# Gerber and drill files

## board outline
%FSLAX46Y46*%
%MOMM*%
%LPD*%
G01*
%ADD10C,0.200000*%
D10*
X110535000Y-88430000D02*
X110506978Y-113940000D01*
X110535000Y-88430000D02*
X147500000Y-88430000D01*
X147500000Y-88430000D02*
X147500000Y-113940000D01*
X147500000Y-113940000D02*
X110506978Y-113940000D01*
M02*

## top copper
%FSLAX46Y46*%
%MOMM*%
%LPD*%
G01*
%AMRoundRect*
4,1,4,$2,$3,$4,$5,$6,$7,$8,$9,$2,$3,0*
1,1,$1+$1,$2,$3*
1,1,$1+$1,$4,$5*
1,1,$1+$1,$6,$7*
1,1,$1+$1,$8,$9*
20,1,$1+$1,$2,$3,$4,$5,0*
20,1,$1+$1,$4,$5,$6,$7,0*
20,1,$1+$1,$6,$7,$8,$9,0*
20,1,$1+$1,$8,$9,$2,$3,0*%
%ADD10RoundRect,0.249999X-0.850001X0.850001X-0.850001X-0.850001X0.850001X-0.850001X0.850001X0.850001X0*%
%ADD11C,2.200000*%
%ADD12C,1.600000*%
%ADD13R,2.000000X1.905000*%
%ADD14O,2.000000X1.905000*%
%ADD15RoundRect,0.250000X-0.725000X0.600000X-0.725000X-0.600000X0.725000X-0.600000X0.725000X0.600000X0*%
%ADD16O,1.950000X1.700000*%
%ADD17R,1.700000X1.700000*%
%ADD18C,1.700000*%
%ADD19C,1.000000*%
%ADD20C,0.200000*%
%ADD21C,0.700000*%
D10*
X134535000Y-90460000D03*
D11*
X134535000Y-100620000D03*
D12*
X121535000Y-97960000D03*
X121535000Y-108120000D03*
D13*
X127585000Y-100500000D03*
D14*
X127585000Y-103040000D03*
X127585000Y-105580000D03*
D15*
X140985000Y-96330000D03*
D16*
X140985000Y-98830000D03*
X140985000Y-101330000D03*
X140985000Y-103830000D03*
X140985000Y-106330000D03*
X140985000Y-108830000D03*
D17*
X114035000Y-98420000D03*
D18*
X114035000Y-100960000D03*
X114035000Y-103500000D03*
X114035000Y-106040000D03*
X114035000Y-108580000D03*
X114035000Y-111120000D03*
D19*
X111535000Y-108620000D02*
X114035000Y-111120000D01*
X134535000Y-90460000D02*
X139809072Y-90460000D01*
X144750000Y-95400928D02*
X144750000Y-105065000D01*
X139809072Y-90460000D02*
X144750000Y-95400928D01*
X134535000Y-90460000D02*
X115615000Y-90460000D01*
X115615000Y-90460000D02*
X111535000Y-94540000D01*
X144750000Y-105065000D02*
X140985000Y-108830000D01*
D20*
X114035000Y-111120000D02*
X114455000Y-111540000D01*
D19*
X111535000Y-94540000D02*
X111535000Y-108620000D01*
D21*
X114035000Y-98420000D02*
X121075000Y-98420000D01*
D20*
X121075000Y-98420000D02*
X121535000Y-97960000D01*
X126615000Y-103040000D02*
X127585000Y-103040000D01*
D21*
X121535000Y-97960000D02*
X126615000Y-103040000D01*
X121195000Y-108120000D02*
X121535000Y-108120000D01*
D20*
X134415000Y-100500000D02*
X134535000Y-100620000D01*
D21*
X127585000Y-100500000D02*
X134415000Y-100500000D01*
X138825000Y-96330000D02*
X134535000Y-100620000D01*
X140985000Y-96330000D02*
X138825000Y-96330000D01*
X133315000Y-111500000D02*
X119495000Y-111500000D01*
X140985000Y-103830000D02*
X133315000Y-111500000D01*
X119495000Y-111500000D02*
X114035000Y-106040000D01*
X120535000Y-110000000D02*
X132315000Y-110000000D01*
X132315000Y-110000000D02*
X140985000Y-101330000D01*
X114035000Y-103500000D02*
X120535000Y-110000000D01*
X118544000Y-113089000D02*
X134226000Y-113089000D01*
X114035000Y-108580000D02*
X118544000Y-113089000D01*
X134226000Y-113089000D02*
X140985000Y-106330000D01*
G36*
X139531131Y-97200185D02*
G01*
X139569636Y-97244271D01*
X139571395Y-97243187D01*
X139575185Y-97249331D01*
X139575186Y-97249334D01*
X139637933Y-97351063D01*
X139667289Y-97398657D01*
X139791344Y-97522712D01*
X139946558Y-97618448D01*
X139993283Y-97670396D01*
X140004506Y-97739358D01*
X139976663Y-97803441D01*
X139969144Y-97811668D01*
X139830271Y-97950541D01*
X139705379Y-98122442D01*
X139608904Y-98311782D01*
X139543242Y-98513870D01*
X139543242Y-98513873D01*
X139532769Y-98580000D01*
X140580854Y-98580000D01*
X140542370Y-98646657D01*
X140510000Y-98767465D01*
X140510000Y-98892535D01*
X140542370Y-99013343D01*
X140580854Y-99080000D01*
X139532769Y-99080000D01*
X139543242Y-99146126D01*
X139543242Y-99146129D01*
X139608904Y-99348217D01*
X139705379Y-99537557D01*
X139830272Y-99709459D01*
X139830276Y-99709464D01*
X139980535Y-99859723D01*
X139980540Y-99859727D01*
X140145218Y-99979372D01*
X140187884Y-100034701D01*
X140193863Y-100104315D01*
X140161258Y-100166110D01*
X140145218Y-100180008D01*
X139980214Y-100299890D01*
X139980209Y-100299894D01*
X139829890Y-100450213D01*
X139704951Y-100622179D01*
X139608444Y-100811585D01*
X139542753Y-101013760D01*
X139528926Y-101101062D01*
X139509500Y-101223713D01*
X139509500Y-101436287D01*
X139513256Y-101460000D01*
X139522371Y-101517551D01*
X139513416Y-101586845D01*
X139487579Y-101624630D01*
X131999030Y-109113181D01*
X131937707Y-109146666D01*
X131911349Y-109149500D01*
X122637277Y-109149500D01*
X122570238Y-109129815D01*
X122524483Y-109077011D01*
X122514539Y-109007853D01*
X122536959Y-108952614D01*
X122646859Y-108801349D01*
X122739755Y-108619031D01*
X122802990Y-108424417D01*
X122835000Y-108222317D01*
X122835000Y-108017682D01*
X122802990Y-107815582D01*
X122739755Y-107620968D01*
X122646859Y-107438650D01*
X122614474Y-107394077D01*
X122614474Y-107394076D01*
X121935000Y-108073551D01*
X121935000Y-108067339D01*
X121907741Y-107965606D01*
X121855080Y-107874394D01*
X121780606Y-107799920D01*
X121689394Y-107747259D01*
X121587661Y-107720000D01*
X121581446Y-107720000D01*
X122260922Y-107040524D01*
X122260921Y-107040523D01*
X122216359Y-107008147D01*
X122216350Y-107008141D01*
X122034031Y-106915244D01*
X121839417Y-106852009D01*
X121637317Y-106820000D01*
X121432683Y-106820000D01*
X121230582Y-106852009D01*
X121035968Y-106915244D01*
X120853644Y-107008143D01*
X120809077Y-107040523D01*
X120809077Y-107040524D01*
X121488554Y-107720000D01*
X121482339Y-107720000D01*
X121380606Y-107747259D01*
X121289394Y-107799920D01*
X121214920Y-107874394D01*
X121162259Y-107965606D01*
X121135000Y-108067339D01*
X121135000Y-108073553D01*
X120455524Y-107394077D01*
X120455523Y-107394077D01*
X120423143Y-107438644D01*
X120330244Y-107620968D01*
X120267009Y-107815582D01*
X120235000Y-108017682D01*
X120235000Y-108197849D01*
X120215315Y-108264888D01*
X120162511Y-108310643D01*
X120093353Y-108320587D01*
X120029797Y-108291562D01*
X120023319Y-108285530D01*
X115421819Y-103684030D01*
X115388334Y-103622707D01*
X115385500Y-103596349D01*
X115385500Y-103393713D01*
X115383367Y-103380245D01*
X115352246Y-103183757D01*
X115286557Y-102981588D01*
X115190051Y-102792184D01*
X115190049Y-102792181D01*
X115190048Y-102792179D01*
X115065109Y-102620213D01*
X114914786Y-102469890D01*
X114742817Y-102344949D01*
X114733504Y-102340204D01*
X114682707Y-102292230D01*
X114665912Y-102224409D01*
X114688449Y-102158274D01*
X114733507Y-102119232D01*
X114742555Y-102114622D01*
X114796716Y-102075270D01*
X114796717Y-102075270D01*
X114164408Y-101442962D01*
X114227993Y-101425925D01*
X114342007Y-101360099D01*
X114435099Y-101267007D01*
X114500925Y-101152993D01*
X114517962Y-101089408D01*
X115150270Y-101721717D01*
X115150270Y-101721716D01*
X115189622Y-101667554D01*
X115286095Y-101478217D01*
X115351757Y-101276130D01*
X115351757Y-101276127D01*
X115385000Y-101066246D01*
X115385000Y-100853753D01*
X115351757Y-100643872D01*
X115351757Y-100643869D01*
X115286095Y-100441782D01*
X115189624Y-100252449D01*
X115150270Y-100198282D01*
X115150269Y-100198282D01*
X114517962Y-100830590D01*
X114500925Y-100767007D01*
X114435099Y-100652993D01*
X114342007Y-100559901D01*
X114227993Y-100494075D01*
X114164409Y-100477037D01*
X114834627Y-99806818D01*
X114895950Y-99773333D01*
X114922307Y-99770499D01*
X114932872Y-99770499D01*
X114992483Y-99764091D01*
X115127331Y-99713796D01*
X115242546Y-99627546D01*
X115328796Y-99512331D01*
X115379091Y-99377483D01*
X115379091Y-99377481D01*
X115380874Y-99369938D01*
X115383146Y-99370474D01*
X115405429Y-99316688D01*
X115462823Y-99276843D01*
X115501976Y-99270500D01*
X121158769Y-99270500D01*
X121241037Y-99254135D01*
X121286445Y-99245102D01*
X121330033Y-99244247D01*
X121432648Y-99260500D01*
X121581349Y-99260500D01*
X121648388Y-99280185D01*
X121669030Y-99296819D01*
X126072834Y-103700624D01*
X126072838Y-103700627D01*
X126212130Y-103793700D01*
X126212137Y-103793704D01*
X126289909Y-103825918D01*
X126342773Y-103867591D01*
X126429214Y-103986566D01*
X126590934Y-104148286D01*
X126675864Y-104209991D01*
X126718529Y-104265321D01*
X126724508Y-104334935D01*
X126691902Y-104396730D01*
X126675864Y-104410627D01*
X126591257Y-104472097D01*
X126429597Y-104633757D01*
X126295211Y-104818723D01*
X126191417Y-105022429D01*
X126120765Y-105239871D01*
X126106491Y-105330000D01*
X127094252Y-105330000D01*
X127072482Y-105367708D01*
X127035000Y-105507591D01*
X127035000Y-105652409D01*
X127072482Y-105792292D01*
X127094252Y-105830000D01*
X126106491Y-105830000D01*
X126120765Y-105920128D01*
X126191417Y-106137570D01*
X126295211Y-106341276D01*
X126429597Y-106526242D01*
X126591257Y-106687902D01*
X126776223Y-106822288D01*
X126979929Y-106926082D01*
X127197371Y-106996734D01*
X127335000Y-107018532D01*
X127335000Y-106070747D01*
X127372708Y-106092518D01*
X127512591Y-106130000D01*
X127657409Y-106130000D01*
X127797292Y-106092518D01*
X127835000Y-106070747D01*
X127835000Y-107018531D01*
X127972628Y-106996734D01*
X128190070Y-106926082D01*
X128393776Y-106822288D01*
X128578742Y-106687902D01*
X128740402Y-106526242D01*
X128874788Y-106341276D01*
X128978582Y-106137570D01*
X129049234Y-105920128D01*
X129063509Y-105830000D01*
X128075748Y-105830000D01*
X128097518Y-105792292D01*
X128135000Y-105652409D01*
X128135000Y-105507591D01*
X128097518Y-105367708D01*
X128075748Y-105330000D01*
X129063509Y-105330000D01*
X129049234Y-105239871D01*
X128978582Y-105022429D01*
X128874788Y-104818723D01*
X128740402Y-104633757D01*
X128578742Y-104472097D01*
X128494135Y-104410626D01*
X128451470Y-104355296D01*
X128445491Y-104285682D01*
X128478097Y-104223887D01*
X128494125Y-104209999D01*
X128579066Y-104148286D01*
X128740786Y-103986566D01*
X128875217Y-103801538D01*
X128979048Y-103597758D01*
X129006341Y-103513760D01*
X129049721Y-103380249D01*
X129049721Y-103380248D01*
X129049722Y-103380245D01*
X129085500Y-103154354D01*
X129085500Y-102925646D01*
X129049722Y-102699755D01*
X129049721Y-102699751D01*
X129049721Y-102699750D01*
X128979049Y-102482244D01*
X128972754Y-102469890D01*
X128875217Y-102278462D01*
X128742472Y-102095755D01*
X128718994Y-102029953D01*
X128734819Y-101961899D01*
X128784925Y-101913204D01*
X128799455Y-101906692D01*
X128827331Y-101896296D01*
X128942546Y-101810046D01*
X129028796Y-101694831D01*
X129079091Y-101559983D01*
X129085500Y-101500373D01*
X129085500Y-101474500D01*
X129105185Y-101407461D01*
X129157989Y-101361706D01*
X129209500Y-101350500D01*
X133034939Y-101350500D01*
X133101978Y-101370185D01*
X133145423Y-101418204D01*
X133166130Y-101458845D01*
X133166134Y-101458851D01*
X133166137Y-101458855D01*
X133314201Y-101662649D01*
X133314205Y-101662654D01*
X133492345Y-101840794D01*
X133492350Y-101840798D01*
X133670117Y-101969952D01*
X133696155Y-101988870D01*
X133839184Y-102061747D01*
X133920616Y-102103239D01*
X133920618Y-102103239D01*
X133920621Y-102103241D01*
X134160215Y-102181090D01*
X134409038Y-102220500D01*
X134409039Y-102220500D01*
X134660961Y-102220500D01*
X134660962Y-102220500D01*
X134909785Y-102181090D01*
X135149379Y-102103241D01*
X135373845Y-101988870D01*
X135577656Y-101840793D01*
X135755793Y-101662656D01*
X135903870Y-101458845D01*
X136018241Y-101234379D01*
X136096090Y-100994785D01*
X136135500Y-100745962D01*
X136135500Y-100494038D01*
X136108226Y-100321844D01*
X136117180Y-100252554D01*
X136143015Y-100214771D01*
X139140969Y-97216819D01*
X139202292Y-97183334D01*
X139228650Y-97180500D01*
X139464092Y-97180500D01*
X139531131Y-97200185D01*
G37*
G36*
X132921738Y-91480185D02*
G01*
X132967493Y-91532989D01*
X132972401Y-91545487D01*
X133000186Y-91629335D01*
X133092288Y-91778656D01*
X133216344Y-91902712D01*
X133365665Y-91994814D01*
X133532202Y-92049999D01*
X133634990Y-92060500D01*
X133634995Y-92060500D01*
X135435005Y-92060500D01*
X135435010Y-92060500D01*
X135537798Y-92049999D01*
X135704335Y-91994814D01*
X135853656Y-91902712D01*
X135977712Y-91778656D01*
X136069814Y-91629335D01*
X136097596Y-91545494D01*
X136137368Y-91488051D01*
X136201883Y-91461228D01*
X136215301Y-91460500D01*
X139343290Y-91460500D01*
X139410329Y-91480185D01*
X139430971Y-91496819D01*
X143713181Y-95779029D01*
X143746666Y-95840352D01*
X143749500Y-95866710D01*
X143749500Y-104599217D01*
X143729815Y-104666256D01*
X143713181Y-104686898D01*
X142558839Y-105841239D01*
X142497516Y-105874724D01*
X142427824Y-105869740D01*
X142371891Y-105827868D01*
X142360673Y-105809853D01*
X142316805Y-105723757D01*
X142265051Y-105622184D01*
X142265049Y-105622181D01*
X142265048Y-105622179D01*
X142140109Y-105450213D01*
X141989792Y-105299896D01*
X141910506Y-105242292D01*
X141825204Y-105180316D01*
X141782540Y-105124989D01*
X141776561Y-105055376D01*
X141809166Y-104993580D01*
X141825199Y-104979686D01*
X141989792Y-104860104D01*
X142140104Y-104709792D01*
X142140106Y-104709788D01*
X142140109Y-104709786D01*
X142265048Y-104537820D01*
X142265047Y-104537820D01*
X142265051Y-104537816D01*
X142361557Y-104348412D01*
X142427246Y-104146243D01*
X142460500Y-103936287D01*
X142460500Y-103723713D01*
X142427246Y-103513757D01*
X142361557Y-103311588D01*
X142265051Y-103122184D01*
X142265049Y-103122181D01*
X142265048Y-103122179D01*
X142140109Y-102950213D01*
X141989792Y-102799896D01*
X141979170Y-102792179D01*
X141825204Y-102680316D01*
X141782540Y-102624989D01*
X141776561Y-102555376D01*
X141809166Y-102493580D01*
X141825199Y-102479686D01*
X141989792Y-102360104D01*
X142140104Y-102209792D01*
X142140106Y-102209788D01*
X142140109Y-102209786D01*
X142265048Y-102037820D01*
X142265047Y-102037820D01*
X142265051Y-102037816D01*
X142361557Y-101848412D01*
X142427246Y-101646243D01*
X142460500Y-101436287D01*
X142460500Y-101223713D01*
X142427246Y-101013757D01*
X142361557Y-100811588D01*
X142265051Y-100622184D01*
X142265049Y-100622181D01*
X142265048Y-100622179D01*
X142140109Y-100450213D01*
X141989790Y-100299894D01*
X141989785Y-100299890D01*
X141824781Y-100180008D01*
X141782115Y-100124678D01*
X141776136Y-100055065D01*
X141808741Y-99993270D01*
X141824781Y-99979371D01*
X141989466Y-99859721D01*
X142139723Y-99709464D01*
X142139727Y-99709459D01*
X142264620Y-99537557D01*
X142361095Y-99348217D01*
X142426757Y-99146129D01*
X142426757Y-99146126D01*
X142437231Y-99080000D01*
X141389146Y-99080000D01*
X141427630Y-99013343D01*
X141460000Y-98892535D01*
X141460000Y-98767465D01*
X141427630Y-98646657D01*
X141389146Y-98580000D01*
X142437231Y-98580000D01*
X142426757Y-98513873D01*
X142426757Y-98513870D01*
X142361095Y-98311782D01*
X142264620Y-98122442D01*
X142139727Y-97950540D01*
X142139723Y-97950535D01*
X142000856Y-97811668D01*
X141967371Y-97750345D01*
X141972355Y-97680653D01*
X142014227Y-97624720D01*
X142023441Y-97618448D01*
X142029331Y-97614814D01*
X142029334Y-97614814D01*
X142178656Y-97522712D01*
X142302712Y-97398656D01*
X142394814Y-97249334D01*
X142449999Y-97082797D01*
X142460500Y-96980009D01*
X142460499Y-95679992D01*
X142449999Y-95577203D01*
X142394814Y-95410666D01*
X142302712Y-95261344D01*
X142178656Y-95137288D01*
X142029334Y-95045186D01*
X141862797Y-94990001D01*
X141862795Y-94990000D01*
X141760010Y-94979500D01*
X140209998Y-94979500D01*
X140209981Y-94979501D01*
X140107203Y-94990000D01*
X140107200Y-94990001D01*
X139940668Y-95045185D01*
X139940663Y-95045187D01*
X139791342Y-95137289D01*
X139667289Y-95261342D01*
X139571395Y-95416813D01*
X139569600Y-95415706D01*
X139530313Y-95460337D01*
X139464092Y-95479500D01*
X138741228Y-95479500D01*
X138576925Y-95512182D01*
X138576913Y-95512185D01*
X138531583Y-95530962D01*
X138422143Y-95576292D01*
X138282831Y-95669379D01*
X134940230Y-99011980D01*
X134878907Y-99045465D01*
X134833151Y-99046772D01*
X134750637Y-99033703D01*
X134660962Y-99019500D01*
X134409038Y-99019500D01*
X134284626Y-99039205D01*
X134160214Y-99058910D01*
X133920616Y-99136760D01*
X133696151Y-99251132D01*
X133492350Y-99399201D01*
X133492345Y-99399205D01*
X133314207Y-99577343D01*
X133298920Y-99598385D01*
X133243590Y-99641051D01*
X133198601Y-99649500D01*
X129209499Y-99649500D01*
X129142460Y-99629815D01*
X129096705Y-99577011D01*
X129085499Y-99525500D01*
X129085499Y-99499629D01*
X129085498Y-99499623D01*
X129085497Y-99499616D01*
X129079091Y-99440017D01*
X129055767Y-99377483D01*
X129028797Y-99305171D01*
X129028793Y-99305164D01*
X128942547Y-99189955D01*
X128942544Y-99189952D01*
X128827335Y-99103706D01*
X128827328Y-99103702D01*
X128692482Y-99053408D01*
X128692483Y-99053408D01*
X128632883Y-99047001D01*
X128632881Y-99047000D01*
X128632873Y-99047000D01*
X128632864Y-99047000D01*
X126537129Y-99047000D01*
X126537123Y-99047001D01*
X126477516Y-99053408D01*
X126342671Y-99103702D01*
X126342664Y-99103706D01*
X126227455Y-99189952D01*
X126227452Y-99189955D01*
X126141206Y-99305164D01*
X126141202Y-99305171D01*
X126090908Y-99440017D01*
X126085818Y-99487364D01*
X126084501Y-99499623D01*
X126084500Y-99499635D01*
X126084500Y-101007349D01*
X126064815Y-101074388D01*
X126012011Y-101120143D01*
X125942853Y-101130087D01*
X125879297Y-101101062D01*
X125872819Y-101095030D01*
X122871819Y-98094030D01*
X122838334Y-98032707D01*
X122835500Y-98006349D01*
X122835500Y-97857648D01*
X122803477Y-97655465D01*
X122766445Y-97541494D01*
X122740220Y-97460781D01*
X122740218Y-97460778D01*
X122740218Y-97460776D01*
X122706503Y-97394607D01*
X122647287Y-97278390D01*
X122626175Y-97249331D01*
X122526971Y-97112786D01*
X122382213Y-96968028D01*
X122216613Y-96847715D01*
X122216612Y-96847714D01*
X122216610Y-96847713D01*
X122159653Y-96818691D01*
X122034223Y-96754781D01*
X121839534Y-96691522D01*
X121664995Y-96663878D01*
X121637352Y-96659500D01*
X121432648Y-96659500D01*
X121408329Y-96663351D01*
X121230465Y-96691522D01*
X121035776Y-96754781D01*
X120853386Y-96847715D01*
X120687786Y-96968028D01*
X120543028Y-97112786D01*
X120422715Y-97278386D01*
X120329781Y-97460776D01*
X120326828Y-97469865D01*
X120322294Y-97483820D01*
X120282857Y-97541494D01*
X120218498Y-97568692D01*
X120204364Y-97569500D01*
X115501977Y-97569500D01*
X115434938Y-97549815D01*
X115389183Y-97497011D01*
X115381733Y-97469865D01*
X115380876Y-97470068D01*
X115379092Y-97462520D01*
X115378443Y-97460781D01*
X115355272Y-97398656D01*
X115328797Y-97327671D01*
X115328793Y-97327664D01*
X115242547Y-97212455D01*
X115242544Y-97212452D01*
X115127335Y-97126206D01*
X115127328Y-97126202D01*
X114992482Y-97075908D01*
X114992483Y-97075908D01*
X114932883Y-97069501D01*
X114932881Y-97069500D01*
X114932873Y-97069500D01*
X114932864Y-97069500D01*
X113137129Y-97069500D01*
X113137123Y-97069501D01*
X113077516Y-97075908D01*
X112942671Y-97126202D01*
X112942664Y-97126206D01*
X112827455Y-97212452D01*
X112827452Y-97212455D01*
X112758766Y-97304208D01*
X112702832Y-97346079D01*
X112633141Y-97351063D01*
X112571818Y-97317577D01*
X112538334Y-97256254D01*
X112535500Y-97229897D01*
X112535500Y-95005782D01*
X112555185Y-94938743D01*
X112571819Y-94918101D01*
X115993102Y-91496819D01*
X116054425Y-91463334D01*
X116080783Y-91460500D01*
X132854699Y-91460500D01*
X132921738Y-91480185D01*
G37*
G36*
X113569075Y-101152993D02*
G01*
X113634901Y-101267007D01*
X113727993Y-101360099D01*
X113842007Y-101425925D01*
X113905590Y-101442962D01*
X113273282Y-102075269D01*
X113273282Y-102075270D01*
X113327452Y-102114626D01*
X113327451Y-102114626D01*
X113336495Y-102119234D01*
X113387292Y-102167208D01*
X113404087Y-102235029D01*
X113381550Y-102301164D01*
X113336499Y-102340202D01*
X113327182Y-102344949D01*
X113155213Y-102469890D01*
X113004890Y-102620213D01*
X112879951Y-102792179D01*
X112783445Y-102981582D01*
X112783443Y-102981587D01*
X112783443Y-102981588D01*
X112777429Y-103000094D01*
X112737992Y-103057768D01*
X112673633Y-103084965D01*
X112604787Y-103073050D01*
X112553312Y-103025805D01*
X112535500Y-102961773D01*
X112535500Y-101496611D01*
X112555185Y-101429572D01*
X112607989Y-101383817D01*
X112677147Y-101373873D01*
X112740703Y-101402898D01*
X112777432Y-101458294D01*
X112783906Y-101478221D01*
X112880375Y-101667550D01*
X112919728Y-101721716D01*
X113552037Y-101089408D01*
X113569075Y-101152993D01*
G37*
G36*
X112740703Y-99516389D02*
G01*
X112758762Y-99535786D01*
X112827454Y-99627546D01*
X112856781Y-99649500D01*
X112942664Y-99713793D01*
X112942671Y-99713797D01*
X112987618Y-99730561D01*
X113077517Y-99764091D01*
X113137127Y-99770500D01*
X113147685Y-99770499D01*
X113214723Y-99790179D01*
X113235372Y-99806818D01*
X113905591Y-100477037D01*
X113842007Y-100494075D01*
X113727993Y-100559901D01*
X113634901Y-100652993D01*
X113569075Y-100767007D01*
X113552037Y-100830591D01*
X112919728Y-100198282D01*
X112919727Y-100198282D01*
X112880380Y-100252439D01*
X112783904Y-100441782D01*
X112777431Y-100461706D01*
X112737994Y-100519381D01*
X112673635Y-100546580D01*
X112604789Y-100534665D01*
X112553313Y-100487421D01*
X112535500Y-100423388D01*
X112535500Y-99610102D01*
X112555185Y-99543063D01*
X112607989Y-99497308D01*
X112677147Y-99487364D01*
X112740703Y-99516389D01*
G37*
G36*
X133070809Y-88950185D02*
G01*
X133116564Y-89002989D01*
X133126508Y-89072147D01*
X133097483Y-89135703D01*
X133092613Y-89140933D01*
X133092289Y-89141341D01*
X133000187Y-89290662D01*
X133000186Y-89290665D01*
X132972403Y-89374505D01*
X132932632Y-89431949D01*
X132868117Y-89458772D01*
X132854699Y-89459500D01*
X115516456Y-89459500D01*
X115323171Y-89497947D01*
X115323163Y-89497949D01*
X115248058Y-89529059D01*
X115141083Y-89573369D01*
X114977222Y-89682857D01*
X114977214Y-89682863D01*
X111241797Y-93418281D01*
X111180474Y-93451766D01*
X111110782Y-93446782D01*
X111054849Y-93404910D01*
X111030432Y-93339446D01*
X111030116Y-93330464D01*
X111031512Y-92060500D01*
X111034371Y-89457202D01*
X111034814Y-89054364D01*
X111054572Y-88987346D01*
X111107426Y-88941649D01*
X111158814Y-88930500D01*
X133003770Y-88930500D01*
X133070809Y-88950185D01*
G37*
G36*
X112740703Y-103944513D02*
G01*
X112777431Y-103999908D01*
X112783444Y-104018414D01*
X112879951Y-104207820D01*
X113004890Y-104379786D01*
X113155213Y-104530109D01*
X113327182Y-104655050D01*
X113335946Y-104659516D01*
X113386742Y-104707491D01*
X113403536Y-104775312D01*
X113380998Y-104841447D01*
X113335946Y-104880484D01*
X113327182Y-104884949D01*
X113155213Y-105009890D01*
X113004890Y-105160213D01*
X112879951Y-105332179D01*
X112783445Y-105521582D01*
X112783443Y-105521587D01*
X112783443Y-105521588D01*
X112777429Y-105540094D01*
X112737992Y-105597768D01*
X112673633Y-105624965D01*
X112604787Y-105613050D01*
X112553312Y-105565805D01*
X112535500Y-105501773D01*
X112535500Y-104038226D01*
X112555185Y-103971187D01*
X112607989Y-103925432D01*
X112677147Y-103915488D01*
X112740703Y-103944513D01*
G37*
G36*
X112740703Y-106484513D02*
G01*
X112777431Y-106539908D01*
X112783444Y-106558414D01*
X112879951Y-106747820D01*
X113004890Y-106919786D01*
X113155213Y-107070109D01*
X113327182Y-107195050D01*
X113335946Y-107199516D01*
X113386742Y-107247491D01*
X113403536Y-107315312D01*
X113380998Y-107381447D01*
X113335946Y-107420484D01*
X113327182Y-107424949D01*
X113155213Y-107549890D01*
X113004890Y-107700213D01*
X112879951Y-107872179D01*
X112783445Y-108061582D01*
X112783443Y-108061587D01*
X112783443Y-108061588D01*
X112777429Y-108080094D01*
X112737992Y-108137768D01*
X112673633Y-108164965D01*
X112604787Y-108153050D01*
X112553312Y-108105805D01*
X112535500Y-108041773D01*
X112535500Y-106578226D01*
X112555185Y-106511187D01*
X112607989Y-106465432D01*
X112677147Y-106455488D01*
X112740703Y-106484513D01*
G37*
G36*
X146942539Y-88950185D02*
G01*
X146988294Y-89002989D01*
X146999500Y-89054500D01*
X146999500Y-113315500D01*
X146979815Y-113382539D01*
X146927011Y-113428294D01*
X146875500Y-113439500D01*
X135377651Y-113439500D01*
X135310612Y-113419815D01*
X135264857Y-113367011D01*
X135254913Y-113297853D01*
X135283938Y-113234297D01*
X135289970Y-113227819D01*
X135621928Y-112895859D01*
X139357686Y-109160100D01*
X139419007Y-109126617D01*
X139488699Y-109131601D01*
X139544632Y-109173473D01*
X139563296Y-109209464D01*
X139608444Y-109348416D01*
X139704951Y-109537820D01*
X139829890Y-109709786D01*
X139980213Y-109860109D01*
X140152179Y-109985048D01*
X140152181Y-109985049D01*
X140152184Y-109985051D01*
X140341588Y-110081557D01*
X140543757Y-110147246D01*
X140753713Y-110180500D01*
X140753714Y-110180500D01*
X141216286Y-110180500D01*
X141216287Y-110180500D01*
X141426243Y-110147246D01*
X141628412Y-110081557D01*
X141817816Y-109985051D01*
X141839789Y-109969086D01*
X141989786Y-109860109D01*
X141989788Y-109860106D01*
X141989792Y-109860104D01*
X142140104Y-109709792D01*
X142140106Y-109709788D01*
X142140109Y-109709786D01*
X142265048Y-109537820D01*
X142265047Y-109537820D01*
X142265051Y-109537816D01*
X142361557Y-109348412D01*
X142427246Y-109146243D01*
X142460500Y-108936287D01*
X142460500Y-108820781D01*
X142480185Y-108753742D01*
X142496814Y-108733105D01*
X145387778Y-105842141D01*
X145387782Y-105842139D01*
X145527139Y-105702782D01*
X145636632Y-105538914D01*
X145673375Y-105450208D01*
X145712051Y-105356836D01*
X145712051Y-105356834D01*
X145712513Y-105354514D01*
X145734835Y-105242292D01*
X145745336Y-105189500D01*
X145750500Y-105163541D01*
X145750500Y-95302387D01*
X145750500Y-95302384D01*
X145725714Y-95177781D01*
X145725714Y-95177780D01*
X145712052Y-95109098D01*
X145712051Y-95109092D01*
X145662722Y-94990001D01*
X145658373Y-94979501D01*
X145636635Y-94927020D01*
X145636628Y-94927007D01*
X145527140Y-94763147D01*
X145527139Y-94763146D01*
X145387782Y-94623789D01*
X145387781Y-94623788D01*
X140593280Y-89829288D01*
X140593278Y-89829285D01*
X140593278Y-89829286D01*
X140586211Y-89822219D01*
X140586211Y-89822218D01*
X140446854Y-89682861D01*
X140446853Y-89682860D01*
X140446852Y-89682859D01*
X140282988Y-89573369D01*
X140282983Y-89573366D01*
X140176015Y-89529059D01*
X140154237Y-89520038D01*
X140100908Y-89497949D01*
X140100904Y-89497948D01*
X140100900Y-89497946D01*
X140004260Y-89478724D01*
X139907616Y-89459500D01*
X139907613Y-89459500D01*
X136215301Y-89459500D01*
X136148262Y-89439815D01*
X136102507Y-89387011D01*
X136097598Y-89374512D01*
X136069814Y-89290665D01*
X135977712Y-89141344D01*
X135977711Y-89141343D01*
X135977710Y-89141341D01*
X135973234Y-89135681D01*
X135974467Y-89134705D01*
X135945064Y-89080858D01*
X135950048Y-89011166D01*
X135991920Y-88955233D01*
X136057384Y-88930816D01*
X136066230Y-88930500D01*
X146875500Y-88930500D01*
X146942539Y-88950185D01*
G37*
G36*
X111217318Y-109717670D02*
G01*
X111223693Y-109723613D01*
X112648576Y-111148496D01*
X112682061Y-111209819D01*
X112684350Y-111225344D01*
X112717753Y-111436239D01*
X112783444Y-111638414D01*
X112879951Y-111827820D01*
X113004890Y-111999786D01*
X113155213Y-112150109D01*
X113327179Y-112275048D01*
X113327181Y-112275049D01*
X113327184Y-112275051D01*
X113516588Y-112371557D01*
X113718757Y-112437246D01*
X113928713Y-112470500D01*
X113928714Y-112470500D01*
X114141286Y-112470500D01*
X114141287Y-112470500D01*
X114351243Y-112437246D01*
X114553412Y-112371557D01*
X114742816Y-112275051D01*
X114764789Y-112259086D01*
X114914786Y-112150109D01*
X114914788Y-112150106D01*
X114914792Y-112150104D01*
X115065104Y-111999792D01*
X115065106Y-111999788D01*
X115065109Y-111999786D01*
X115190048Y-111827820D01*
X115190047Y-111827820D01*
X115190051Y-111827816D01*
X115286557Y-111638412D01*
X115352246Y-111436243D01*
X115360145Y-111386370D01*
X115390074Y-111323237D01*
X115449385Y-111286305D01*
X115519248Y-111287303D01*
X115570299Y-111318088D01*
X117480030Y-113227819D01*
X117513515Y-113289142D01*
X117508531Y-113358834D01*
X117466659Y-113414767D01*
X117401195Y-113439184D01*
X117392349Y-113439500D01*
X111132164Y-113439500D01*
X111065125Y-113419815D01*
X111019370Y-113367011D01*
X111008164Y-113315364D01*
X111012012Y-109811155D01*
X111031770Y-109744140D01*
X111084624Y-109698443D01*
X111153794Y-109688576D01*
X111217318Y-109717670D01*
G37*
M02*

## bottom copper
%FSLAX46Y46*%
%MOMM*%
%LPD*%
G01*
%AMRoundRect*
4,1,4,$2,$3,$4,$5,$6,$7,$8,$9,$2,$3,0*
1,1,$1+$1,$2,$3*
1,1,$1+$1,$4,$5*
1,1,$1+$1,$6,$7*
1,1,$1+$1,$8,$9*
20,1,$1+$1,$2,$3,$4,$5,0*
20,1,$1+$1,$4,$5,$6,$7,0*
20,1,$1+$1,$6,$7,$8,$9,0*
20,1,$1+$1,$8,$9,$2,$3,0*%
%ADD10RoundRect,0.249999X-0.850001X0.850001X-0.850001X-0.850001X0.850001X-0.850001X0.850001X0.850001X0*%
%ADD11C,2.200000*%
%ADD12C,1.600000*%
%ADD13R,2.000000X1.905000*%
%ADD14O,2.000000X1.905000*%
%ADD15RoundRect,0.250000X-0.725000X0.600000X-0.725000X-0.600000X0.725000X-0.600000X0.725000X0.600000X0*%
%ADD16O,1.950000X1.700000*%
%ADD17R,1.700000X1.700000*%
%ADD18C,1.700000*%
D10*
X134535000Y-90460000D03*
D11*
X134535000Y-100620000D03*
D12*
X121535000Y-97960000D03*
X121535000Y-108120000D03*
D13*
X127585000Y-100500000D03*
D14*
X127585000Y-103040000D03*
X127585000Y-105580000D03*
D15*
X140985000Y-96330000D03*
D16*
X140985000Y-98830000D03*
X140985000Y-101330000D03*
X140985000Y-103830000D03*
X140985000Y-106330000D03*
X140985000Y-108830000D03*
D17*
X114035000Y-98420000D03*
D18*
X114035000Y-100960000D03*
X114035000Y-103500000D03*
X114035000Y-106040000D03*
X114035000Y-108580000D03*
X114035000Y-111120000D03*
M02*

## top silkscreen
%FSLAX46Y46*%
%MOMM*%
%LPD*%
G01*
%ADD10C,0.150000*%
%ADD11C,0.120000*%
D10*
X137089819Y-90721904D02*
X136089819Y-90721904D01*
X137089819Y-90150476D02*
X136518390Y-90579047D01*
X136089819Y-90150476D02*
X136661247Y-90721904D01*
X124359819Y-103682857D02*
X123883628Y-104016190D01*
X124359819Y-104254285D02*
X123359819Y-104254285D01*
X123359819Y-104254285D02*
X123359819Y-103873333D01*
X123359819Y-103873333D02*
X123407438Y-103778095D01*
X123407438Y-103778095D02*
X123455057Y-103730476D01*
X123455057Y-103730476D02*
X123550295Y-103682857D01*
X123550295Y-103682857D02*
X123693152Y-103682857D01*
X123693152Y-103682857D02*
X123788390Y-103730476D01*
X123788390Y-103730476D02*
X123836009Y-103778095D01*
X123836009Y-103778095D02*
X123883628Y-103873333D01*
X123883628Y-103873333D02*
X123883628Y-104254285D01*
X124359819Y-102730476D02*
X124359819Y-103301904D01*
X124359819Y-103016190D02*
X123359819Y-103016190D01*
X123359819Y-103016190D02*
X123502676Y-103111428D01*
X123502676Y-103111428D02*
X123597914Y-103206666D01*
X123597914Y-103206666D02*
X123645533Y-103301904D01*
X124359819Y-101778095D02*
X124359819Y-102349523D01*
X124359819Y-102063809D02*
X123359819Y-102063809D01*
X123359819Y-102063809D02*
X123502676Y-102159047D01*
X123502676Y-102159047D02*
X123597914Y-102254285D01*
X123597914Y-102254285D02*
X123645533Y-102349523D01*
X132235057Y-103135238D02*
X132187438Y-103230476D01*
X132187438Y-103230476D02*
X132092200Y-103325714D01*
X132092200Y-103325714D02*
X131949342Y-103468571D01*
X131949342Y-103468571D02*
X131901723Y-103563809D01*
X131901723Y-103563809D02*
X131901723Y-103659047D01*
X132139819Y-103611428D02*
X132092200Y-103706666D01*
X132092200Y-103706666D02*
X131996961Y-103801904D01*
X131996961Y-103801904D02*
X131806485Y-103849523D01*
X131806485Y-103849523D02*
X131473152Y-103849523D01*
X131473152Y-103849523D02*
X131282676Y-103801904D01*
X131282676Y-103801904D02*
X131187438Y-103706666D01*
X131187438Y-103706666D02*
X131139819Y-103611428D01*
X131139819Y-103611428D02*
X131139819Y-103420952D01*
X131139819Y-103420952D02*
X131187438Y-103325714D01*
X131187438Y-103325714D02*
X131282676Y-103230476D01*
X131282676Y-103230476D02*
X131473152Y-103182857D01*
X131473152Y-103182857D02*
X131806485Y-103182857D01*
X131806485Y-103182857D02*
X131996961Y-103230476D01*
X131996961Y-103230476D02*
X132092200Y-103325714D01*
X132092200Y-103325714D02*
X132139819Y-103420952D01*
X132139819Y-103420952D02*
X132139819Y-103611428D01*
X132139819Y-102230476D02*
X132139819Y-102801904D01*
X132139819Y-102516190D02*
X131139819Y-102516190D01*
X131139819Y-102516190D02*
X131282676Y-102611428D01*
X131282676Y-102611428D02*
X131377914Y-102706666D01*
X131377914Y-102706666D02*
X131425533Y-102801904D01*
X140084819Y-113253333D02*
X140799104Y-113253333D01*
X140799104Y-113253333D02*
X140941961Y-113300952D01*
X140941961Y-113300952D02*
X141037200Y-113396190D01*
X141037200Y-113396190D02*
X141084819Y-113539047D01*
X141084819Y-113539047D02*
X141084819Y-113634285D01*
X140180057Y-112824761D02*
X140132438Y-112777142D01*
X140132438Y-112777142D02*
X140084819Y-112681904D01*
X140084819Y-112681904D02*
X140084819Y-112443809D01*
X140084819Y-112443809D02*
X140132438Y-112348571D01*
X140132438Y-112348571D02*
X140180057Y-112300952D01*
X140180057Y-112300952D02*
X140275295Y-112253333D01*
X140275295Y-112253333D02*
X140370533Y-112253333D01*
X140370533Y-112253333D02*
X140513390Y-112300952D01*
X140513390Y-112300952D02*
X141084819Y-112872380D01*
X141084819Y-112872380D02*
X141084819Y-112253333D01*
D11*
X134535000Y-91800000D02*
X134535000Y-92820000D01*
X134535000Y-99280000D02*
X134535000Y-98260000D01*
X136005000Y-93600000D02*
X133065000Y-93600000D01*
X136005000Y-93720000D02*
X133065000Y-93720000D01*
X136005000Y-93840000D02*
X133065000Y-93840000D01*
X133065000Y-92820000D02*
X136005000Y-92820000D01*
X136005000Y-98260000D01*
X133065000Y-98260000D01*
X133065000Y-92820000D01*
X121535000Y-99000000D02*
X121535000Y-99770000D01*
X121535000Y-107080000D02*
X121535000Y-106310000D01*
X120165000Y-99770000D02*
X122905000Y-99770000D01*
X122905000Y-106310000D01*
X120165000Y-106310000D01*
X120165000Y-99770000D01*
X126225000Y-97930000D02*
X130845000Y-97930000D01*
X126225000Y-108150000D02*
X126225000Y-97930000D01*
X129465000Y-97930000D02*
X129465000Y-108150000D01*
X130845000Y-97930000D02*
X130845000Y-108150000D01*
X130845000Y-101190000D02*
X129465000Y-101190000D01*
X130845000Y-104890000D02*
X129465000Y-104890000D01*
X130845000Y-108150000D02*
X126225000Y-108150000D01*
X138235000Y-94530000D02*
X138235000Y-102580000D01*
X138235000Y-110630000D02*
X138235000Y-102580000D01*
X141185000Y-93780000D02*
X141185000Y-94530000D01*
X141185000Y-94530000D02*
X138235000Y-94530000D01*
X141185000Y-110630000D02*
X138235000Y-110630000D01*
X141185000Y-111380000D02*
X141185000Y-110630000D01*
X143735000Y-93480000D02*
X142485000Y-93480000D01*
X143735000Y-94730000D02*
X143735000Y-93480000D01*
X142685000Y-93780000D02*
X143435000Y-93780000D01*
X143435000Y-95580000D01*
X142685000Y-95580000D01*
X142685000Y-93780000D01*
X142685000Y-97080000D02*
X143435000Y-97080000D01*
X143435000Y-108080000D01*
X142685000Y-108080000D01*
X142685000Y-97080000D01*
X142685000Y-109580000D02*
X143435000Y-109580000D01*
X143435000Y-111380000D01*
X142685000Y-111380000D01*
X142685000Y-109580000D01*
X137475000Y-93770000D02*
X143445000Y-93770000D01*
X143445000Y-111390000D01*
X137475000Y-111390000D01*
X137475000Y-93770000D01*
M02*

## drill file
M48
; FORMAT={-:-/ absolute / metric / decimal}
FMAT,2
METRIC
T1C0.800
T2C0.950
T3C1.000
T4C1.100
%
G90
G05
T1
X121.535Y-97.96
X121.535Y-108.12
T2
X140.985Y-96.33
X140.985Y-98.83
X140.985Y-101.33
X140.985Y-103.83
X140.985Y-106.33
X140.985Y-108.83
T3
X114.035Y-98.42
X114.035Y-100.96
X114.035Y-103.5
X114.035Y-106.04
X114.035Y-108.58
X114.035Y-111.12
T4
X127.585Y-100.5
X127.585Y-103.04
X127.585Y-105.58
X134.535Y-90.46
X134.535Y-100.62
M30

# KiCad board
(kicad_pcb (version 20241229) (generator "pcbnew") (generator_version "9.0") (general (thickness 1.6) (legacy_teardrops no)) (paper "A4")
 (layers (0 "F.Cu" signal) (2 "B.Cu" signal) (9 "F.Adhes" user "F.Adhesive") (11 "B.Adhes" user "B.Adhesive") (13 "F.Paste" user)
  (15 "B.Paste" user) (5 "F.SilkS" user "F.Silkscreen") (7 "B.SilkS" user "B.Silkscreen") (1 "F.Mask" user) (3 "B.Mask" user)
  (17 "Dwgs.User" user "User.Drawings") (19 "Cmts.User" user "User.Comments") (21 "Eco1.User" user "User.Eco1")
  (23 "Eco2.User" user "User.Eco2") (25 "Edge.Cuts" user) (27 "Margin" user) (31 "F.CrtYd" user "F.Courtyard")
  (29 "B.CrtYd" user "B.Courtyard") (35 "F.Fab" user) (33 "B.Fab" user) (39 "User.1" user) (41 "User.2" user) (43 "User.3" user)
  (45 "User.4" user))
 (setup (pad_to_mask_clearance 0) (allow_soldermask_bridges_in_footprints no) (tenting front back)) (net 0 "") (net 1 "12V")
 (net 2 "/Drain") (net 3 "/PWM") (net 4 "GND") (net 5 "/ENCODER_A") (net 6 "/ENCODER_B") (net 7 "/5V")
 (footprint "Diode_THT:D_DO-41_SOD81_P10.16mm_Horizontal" (layer "F.Cu") (at 134.535 90.46 -90)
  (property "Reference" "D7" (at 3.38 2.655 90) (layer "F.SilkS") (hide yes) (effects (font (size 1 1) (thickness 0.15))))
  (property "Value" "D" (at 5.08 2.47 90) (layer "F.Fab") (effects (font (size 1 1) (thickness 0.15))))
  (fp_line (start 1.34 0) (end 2.36 0) (stroke (width 0.12) (type solid)) (layer "F.SilkS"))
  (fp_line (start 8.82 0) (end 7.8 0) (stroke (width 0.12) (type solid)) (layer "F.SilkS"))
  (fp_line (start 3.14 -1.47) (end 3.14 1.47) (stroke (width 0.12) (type solid)) (layer "F.SilkS"))
  (fp_line (start 3.26 -1.47) (end 3.26 1.47) (stroke (width 0.12) (type solid)) (layer "F.SilkS"))
  (fp_line (start 3.38 -1.47) (end 3.38 1.47) (stroke (width 0.12) (type solid)) (layer "F.SilkS"))
  (fp_rect (start 2.36 -1.47) (end 7.8 1.47) (stroke (width 0.12) (type solid)) (fill no) (layer "F.SilkS"))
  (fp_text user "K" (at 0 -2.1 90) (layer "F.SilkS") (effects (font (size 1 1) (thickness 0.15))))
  (pad "1" thru_hole roundrect (at 0 0 270) (size 2.2 2.2) (drill 1.1) (layers "*.Cu" "*.Mask") (remove_unused_layers no)
   (roundrect_rratio 0.113636) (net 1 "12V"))
  (pad "2" thru_hole circle (at 10.16 0 270) (size 2.2 2.2) (drill 1.1) (layers "*.Cu" "*.Mask") (remove_unused_layers no) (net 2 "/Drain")))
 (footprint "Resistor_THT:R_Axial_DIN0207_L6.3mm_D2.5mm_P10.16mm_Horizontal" (layer "F.Cu") (at 121.535 97.96 -90)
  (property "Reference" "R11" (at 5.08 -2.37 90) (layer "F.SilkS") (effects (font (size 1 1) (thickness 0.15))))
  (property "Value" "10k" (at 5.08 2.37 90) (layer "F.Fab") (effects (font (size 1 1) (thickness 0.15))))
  (fp_line (start 1.04 0) (end 1.81 0) (stroke (width 0.12) (type solid)) (layer "F.SilkS"))
  (fp_line (start 9.12 0) (end 8.35 0) (stroke (width 0.12) (type solid)) (layer "F.SilkS"))
  (fp_rect (start 1.81 -1.37) (end 8.35 1.37) (stroke (width 0.12) (type solid)) (fill no) (layer "F.SilkS"))
  (pad "1" thru_hole circle (at 0 0 270) (size 1.6 1.6) (drill 0.8) (layers "*.Cu" "*.Mask") (remove_unused_layers no) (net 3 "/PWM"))
  (pad "2" thru_hole circle (at 10.16 0 270) (size 1.6 1.6) (drill 0.8) (layers "*.Cu" "*.Mask") (remove_unused_layers no) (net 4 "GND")))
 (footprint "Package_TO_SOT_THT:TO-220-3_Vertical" (layer "F.Cu") (at 127.585 100.5 -90)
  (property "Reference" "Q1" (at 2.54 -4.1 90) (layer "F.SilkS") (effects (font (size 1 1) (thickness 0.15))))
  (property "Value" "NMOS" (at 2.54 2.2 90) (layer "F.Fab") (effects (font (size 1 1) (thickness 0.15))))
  (fp_line (start -2.57 1.36) (end -2.57 -3.26) (stroke (width 0.12) (type solid)) (layer "F.SilkS"))
  (fp_line (start 7.65 1.36) (end -2.57 1.36) (stroke (width 0.12) (type solid)) (layer "F.SilkS"))
  (fp_line (start -2.57 -1.88) (end 7.65 -1.88) (stroke (width 0.12) (type solid)) (layer "F.SilkS"))
  (fp_line (start -2.57 -3.26) (end 7.65 -3.26) (stroke (width 0.12) (type solid)) (layer "F.SilkS"))
  (fp_line (start 0.69 -3.26) (end 0.69 -1.88) (stroke (width 0.12) (type solid)) (layer "F.SilkS"))
  (fp_line (start 4.39 -3.26) (end 4.39 -1.88) (stroke (width 0.12) (type solid)) (layer "F.SilkS"))
  (fp_line (start 7.65 -3.26) (end 7.65 1.36) (stroke (width 0.12) (type solid)) (layer "F.SilkS"))
  (pad "1" thru_hole rect (at 0 0 270) (size 1.905 2) (drill 1.1) (layers "*.Cu" "*.Mask") (remove_unused_layers no) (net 2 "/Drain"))
  (pad "2" thru_hole oval (at 2.54 0 270) (size 1.905 2) (drill 1.1) (layers "*.Cu" "*.Mask") (remove_unused_layers no) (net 3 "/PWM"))
  (pad "3" thru_hole oval (at 5.08 0 270) (size 1.905 2) (drill 1.1) (layers "*.Cu" "*.Mask") (remove_unused_layers no) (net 4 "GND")))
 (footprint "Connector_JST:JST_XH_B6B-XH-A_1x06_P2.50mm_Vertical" (layer "F.Cu") (at 140.985 96.33 -90)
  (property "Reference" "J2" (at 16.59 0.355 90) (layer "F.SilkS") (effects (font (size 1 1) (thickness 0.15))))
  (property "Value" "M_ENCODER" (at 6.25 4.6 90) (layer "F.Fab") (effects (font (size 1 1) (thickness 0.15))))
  (fp_line (start -1.8 2.75) (end 6.25 2.75) (stroke (width 0.12) (type solid)) (layer "F.SilkS"))
  (fp_line (start 14.3 2.75) (end 6.25 2.75) (stroke (width 0.12) (type solid)) (layer "F.SilkS"))
  (fp_line (start -2.55 -0.2) (end -1.8 -0.2) (stroke (width 0.12) (type solid)) (layer "F.SilkS"))
  (fp_line (start -1.8 -0.2) (end -1.8 2.75) (stroke (width 0.12) (type solid)) (layer "F.SilkS"))
  (fp_line (start 14.3 -0.2) (end 14.3 2.75) (stroke (width 0.12) (type solid)) (layer "F.SilkS"))
  (fp_line (start 15.05 -0.2) (end 14.3 -0.2) (stroke (width 0.12) (type solid)) (layer "F.SilkS"))
  (fp_line (start -2.85 -2.75) (end -2.85 -1.5) (stroke (width 0.12) (type solid)) (layer "F.SilkS"))
  (fp_line (start -1.6 -2.75) (end -2.85 -2.75) (stroke (width 0.12) (type solid)) (layer "F.SilkS"))
  (fp_rect (start -2.55 -2.45) (end -0.75 -1.7) (stroke (width 0.12) (type solid)) (fill no) (layer "F.SilkS"))
  (fp_rect (start 0.75 -2.45) (end 11.75 -1.7) (stroke (width 0.12) (type solid)) (fill no) (layer "F.SilkS"))
  (fp_rect (start 13.25 -2.45) (end 15.05 -1.7) (stroke (width 0.12) (type solid)) (fill no) (layer "F.SilkS"))
  (fp_rect (start -2.56 -2.46) (end 15.06 3.51) (stroke (width 0.12) (type solid)) (fill no) (layer "F.SilkS"))
  (pad "1" thru_hole roundrect (at 0 0 270) (size 1.7 1.95) (drill 0.95) (layers "*.Cu" "*.Mask") (remove_unused_layers no)
   (roundrect_rratio 0.147059) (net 2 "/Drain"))
  (pad "2" thru_hole oval (at 2.5 0 270) (size 1.7 1.95) (drill 0.95) (layers "*.Cu" "*.Mask") (remove_unused_layers no) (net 4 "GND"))
  (pad "3" thru_hole oval (at 5 0 270) (size 1.7 1.95) (drill 0.95) (layers "*.Cu" "*.Mask") (remove_unused_layers no) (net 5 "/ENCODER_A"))
  (pad "4" thru_hole oval (at 7.5 0 270) (size 1.7 1.95) (drill 0.95) (layers "*.Cu" "*.Mask") (remove_unused_layers no)
   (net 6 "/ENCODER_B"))
  (pad "5" thru_hole oval (at 10 0 270) (size 1.7 1.95) (drill 0.95) (layers "*.Cu" "*.Mask") (remove_unused_layers no) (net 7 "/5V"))
  (pad "6" thru_hole oval (at 12.5 0 270) (size 1.7 1.95) (drill 0.95) (layers "*.Cu" "*.Mask") (remove_unused_layers no) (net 1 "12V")))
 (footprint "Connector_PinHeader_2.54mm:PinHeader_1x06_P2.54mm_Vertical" (layer "B.Cu") (at 114.035 98.42 180)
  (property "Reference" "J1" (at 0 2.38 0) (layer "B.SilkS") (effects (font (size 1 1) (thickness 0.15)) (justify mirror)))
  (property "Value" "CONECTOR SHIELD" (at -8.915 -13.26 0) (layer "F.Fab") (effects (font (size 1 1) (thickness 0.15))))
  (pad "1" thru_hole rect (at 0 0 180) (size 1.7 1.7) (drill 1) (layers "*.Cu" "*.Mask") (remove_unused_layers no) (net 3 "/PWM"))
  (pad "2" thru_hole circle (at 0 -2.54 180) (size 1.7 1.7) (drill 1) (layers "*.Cu" "*.Mask") (remove_unused_layers no) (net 4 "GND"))
  (pad "3" thru_hole circle (at 0 -5.08 180) (size 1.7 1.7) (drill 1) (layers "*.Cu" "*.Mask") (remove_unused_layers no)
   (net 5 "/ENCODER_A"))
  (pad "4" thru_hole circle (at 0 -7.62 180) (size 1.7 1.7) (drill 1) (layers "*.Cu" "*.Mask") (remove_unused_layers no)
   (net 6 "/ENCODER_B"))
  (pad "5" thru_hole circle (at 0 -10.16 180) (size 1.7 1.7) (drill 1) (layers "*.Cu" "*.Mask") (remove_unused_layers no) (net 7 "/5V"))
  (pad "6" thru_hole circle (at 0 -12.7 180) (size 1.7 1.7) (drill 1) (layers "*.Cu" "*.Mask") (remove_unused_layers no) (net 1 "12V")))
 (gr_line (start 110.535 88.43) (end 110.506978 113.94) (stroke (width 0.2) (type solid)) (layer "Edge.Cuts"))
 (gr_line (start 110.535 88.43) (end 147.5 88.43) (stroke (width 0.2) (type solid)) (layer "Edge.Cuts"))
 (gr_line (start 147.5 88.43) (end 147.5 113.94) (stroke (width 0.2) (type solid)) (layer "Edge.Cuts"))
 (gr_line (start 147.5 113.94) (end 110.506978 113.94) (stroke (width 0.2) (type solid)) (layer "Edge.Cuts"))
 (segment (start 111.535 108.62) (end 114.035 111.12) (width 1) (layer "F.Cu") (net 1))
 (segment (start 134.535 90.46) (end 139.809072 90.46) (width 1) (layer "F.Cu") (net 1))
 (segment (start 144.75 95.400928) (end 144.75 105.065) (width 1) (layer "F.Cu") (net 1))
 (segment (start 139.809072 90.46) (end 144.75 95.400928) (width 1) (layer "F.Cu") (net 1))
 (segment (start 134.535 90.46) (end 115.615 90.46) (width 1) (layer "F.Cu") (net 1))
 (segment (start 115.615 90.46) (end 111.535 94.54) (width 1) (layer "F.Cu") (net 1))
 (segment (start 144.75 105.065) (end 140.985 108.83) (width 1) (layer "F.Cu") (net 1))
 (segment (start 114.035 111.12) (end 114.455 111.54) (width 0.2) (layer "F.Cu") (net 1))
 (segment (start 111.535 94.54) (end 111.535 108.62) (width 1) (layer "F.Cu") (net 1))
 (segment (start 114.035 98.42) (end 121.075 98.42) (width 0.7) (layer "F.Cu") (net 3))
 (segment (start 121.075 98.42) (end 121.535 97.96) (width 0.2) (layer "F.Cu") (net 3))
 (segment (start 126.615 103.04) (end 127.585 103.04) (width 0.2) (layer "F.Cu") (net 3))
 (segment (start 121.535 97.96) (end 126.615 103.04) (width 0.7) (layer "F.Cu") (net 3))
 (segment (start 121.195 108.12) (end 121.535 108.12) (width 0.7) (layer "F.Cu") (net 4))
 (segment (start 134.415 100.5) (end 134.535 100.62) (width 0.2) (layer "F.Cu") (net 2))
 (segment (start 127.585 100.5) (end 134.415 100.5) (width 0.7) (layer "F.Cu") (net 2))
 (segment (start 138.825 96.33) (end 134.535 100.62) (width 0.7) (layer "F.Cu") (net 2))
 (segment (start 140.985 96.33) (end 138.825 96.33) (width 0.7) (layer "F.Cu") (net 2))
 (segment (start 133.315 111.5) (end 119.495 111.5) (width 0.7) (layer "F.Cu") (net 6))
 (segment (start 140.985 103.83) (end 133.315 111.5) (width 0.7) (layer "F.Cu") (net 6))
 (segment (start 119.495 111.5) (end 114.035 106.04) (width 0.7) (layer "F.Cu") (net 6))
 (segment (start 120.535 110) (end 132.315 110) (width 0.7) (layer "F.Cu") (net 5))
 (segment (start 132.315 110) (end 140.985 101.33) (width 0.7) (layer "F.Cu") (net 5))
 (segment (start 114.035 103.5) (end 120.535 110) (width 0.7) (layer "F.Cu") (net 5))
 (segment (start 118.544 113.089) (end 134.226 113.089) (width 0.7) (layer "F.Cu") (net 7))
 (segment (start 114.035 108.58) (end 118.544 113.089) (width 0.7) (layer "F.Cu") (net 7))
 (segment (start 134.226 113.089) (end 140.985 106.33) (width 0.7) (layer "F.Cu") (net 7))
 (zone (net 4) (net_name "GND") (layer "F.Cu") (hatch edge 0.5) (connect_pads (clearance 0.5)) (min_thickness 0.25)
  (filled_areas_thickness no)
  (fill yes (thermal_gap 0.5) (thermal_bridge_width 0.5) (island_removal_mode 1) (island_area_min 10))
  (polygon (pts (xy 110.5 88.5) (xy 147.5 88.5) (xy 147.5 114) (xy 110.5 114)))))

